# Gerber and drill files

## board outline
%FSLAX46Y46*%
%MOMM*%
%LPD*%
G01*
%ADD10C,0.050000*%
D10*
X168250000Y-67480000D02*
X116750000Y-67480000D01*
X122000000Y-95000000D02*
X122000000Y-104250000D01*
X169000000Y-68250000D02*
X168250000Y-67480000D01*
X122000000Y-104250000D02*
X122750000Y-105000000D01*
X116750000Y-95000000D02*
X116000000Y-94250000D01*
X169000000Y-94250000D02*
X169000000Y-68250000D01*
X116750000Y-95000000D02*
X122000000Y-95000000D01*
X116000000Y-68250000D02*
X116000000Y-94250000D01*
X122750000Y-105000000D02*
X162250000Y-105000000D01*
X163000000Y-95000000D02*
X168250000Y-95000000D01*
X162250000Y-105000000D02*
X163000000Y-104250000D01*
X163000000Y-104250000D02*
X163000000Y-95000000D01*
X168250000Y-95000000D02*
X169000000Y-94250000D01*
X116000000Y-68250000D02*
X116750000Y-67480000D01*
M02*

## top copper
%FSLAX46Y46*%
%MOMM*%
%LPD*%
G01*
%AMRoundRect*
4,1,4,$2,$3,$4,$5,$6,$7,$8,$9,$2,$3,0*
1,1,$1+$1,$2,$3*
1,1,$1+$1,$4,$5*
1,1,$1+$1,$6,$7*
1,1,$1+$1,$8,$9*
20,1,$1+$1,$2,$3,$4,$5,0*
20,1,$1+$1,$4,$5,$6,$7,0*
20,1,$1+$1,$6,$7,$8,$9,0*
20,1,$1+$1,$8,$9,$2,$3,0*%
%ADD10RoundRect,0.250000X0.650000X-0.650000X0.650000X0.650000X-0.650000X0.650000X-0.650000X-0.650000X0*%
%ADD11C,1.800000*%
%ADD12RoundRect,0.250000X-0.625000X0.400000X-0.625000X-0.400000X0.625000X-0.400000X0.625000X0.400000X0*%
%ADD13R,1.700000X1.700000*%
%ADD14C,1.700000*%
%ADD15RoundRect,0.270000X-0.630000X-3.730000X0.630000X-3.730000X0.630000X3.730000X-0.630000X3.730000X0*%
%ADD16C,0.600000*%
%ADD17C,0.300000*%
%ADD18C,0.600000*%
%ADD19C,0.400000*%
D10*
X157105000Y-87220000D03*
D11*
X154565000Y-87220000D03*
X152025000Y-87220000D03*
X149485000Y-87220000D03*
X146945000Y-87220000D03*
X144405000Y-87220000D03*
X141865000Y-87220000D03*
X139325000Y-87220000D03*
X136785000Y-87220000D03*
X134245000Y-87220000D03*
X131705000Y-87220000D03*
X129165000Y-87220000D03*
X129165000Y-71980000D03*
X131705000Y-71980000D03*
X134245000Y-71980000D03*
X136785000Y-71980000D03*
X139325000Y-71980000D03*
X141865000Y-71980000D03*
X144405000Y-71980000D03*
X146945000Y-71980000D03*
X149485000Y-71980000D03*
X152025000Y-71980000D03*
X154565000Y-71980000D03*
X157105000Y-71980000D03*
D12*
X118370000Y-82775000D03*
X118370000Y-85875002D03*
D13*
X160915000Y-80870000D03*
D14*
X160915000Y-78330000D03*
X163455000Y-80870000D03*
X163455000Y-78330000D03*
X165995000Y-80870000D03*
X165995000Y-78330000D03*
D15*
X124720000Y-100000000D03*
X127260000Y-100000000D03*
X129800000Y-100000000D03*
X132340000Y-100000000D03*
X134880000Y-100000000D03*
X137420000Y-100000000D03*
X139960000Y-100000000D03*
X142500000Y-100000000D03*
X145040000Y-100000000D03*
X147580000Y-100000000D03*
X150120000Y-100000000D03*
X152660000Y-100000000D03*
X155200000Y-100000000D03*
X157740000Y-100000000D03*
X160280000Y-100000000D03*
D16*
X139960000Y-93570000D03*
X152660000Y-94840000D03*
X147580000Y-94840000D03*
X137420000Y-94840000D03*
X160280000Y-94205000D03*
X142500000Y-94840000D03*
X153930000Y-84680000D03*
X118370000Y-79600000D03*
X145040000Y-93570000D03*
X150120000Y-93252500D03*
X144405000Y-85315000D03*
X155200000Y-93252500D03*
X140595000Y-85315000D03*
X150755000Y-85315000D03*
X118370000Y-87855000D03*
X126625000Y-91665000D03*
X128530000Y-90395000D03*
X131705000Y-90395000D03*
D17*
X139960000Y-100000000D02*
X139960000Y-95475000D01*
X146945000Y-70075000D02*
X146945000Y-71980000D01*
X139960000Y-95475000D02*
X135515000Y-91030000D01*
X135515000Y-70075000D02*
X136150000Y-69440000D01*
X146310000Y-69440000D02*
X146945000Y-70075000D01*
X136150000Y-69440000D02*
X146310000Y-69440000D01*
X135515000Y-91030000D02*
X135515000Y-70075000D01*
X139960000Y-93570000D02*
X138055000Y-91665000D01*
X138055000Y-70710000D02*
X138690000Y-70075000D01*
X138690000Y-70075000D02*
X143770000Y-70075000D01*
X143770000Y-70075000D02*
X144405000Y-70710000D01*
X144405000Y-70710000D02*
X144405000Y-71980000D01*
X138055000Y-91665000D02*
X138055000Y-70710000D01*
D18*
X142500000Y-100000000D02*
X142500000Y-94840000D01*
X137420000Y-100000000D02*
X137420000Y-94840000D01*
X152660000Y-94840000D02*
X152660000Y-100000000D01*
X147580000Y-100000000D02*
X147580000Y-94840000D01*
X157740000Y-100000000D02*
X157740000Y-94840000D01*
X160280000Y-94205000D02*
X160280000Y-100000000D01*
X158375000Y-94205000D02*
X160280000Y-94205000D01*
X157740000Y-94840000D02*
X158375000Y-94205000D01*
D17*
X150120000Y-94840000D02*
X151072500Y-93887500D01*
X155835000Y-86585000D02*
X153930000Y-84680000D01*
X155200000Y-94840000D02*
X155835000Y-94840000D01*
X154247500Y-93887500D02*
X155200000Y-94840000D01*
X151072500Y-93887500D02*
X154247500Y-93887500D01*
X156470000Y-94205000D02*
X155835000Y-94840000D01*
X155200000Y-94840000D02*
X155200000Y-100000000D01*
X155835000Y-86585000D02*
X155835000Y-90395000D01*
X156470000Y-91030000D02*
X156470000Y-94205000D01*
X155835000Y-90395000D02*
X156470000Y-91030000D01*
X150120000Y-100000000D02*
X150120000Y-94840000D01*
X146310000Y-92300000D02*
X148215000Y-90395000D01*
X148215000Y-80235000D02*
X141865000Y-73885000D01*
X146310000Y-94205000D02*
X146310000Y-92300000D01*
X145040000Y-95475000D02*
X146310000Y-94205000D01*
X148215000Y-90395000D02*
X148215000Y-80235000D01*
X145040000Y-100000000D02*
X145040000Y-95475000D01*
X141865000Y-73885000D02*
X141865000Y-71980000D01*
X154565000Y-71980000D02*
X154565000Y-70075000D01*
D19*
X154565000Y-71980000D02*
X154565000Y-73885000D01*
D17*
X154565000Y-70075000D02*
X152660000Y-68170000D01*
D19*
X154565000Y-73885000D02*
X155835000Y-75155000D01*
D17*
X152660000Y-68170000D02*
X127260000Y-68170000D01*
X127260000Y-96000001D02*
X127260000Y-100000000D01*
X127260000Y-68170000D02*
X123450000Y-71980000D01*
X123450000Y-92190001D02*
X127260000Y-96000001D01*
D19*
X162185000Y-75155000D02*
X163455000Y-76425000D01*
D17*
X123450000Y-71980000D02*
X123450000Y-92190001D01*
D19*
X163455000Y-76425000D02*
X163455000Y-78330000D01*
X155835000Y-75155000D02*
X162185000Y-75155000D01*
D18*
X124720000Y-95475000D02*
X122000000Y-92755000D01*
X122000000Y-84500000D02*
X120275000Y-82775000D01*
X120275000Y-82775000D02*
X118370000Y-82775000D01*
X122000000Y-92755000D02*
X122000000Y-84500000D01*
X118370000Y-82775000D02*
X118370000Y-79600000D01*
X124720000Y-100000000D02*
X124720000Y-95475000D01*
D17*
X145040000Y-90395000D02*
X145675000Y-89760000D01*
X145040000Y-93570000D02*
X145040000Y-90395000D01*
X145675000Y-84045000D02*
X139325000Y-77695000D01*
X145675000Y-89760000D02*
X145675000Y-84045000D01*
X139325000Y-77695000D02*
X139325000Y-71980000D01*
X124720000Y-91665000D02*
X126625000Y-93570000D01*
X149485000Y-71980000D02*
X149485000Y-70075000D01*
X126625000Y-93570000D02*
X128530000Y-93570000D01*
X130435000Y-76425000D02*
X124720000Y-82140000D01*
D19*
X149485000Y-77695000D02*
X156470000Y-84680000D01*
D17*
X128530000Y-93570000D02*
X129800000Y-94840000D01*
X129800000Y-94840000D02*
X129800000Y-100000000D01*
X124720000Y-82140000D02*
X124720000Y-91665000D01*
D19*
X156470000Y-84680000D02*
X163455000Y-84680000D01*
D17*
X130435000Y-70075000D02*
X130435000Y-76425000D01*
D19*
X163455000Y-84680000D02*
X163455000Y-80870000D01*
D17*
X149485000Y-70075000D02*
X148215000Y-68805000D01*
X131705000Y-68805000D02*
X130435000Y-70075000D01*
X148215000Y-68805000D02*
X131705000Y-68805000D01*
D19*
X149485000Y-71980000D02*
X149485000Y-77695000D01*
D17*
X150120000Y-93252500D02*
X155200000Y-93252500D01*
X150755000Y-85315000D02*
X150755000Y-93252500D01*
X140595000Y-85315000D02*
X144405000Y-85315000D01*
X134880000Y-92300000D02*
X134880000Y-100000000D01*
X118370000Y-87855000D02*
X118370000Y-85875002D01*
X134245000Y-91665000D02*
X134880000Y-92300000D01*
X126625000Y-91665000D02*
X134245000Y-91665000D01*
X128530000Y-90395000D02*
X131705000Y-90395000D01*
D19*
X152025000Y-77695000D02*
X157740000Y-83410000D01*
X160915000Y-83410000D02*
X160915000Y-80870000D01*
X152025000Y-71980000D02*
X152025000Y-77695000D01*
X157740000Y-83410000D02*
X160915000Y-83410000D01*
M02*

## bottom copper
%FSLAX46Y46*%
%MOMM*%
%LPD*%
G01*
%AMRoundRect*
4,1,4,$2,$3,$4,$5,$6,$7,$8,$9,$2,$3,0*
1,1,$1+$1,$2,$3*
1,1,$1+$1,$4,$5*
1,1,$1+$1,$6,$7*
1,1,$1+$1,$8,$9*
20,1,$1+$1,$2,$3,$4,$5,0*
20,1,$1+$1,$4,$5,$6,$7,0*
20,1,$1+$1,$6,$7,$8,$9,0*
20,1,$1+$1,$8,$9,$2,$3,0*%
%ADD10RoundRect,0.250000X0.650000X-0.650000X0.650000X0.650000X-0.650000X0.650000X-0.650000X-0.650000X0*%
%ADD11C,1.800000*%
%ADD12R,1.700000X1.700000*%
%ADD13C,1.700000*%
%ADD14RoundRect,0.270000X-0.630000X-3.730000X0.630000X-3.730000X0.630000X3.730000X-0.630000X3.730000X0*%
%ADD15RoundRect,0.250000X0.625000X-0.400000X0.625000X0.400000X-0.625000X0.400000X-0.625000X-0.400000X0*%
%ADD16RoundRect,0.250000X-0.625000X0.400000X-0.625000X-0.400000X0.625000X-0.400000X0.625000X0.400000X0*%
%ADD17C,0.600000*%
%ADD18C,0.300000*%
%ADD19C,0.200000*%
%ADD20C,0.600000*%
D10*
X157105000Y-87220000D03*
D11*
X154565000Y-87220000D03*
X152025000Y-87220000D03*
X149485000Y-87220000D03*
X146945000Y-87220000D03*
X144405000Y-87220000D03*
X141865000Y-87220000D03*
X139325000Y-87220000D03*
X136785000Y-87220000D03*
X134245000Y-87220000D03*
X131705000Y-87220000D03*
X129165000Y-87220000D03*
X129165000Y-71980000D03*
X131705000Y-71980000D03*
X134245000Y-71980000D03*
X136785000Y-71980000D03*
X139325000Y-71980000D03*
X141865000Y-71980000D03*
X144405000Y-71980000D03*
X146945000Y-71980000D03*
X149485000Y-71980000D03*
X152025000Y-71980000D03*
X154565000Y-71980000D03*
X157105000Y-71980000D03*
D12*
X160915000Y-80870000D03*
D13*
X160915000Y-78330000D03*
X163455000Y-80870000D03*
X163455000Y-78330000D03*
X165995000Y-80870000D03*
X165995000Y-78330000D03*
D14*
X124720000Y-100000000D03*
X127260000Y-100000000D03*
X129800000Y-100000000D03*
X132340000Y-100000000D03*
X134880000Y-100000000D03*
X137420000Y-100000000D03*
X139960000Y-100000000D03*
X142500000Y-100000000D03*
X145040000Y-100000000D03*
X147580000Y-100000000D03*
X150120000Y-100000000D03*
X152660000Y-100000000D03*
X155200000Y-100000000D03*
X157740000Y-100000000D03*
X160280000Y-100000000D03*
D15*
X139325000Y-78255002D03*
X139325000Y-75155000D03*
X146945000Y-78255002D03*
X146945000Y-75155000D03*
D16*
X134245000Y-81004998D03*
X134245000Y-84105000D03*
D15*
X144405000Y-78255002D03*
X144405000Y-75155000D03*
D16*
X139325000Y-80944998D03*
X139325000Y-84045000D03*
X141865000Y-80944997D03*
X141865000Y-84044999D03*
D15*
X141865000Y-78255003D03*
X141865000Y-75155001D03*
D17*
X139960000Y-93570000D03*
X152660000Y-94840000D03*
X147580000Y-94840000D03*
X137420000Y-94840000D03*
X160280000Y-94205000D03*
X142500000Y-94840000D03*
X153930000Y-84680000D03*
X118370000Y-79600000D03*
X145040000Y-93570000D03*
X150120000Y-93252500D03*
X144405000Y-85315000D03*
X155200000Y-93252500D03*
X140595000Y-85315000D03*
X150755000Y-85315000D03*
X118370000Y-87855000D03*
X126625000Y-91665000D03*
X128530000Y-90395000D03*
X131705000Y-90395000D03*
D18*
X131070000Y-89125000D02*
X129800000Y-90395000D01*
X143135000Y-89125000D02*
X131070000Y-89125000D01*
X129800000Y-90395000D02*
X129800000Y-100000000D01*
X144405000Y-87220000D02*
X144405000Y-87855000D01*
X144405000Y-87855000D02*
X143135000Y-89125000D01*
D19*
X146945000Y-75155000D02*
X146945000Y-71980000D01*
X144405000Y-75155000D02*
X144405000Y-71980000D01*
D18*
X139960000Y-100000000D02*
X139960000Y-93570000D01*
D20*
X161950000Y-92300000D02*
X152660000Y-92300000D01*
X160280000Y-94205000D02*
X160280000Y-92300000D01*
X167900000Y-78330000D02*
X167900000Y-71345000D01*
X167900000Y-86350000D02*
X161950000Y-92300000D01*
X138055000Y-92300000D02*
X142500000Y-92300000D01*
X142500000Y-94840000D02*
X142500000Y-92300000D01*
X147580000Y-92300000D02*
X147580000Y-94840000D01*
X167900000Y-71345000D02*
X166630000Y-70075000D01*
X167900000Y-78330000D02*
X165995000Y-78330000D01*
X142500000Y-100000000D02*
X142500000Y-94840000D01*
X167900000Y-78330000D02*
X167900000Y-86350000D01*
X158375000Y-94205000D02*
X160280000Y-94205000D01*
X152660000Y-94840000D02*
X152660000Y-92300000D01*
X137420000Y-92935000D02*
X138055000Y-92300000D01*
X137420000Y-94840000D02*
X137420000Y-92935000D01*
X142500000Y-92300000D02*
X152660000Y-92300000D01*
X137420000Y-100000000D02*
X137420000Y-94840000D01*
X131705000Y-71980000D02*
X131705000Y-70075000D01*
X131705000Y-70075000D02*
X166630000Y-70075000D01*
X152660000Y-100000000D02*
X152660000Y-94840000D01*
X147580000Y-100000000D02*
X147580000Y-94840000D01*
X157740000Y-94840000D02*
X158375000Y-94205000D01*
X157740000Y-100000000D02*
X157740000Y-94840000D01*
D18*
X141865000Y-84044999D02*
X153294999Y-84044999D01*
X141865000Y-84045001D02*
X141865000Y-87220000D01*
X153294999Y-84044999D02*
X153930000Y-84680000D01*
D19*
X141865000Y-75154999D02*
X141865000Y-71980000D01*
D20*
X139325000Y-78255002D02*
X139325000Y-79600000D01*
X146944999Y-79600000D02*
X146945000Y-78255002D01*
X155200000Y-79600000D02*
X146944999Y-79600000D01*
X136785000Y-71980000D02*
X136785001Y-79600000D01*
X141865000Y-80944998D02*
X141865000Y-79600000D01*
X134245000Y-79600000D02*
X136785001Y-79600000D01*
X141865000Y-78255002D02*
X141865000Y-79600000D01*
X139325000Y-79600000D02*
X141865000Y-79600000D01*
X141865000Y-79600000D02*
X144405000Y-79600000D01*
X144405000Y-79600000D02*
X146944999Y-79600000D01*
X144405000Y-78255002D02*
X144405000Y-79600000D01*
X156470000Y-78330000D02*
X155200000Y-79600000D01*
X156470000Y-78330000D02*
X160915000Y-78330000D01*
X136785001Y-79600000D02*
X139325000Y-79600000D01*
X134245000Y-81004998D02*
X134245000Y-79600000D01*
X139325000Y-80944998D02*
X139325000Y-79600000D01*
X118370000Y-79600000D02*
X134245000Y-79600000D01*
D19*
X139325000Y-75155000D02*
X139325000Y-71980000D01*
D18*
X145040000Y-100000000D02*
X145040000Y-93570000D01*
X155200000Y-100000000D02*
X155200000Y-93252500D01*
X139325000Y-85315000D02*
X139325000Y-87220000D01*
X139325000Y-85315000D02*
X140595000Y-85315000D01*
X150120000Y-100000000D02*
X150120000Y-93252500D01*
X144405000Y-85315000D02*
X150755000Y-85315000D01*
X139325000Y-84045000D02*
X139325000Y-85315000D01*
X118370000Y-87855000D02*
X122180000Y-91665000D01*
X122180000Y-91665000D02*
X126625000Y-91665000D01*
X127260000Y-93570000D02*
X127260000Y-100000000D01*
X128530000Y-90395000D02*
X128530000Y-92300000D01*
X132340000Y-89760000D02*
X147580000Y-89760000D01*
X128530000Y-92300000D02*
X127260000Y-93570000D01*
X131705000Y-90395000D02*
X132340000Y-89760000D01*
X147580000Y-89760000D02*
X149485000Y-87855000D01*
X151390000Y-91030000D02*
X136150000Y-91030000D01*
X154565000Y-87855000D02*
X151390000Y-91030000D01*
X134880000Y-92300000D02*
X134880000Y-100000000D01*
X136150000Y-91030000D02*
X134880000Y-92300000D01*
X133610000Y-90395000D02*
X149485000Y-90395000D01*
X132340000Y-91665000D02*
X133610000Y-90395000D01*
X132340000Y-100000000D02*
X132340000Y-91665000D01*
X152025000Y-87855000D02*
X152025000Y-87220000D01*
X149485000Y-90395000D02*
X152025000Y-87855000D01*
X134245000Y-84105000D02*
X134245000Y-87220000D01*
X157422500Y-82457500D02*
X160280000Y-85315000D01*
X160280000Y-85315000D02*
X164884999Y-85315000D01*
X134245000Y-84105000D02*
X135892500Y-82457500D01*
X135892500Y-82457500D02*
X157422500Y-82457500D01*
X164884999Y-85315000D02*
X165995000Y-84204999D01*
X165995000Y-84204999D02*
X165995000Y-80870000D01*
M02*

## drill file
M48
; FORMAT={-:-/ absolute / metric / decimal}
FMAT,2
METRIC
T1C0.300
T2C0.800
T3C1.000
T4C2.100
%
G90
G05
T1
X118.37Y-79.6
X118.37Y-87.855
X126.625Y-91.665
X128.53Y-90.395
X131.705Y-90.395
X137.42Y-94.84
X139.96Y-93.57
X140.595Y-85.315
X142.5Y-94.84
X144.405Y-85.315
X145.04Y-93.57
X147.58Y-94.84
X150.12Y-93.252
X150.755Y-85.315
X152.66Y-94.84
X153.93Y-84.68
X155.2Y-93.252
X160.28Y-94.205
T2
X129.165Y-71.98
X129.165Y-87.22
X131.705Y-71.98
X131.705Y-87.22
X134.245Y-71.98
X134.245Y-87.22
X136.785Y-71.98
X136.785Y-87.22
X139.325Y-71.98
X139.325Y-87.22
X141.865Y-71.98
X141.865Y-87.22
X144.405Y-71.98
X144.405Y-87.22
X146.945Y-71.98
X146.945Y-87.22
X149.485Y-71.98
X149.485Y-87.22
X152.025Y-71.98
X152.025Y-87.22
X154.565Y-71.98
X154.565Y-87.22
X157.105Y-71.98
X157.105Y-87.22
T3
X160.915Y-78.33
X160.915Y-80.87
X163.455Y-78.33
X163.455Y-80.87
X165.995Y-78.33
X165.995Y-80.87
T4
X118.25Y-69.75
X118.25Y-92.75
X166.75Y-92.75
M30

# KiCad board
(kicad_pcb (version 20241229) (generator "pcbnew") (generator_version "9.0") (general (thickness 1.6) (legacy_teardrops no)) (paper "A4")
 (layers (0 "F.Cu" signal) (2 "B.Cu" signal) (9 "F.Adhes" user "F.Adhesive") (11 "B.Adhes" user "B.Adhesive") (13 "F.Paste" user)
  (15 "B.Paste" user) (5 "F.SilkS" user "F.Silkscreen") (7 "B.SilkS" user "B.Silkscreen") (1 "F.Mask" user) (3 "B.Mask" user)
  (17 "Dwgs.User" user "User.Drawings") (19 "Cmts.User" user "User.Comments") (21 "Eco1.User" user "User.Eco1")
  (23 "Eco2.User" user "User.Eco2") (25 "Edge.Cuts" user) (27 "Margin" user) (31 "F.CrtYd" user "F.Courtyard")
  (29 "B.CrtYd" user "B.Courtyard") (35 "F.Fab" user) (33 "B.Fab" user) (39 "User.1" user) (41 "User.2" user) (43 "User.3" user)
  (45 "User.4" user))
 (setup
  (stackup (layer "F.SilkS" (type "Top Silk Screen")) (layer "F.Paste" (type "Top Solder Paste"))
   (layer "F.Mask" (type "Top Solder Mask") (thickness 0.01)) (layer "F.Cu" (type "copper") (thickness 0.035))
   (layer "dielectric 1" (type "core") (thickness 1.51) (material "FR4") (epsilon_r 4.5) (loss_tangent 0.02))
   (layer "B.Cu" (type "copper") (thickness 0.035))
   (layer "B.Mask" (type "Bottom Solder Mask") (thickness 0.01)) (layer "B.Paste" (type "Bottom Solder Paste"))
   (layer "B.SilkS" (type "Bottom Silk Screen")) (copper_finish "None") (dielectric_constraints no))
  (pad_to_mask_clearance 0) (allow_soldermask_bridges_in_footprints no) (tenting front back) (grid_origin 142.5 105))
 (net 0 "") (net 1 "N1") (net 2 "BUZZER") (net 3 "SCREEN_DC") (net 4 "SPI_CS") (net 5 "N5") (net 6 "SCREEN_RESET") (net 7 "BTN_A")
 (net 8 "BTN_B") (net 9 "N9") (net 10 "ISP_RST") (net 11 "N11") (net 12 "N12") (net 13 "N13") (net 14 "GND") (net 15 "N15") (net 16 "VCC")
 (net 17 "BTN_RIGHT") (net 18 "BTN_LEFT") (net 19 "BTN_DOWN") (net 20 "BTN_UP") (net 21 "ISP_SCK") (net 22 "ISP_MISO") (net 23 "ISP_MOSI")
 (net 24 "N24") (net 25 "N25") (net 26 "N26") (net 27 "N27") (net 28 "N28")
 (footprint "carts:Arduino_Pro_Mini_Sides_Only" (layer "F.Cu") (at 141.865 79.6 90)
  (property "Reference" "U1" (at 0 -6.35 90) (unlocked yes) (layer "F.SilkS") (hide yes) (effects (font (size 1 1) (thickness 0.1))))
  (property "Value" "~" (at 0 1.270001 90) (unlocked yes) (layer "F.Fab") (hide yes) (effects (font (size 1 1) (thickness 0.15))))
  (pad "1" thru_hole roundrect (at -7.62 15.24 90) (size 1.8 1.8) (drill 0.8) (layers "*.Cu" "*.Mask") (remove_unused_layers no)
   (roundrect_rratio 0.1388888889) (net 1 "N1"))
  (pad "2" thru_hole circle (at -7.62 12.7 90) (size 1.8 1.8) (drill 0.8) (layers "*.Cu" "*.Mask") (remove_unused_layers no)
   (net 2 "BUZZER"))
  (pad "3" thru_hole circle (at -7.62 10.16 90) (size 1.8 1.8) (drill 0.8) (layers "*.Cu" "*.Mask") (remove_unused_layers no)
   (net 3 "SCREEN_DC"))
  (pad "4" thru_hole circle (at -7.62 7.62 90) (size 1.8 1.8) (drill 0.8) (layers "*.Cu" "*.Mask") (remove_unused_layers no)
   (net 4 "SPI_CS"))
  (pad "5" thru_hole circle (at -7.62 5.08 90) (size 1.8 1.8) (drill 0.8) (layers "*.Cu" "*.Mask") (remove_unused_layers no) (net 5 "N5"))
  (pad "6" thru_hole circle (at -7.62 2.54 90) (size 1.8 1.8) (drill 0.8) (layers "*.Cu" "*.Mask") (remove_unused_layers no)
   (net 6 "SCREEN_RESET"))
  (pad "7" thru_hole circle (at -7.62 0 90) (size 1.8 1.8) (drill 0.8) (layers "*.Cu" "*.Mask") (remove_unused_layers no) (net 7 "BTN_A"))
  (pad "8" thru_hole circle (at -7.62 -2.54 90) (size 1.8 1.8) (drill 0.8) (layers "*.Cu" "*.Mask") (remove_unused_layers no)
   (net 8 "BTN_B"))
  (pad "9" thru_hole circle (at -7.62 -5.08 90) (size 1.8 1.8) (drill 0.8) (layers "*.Cu" "*.Mask") (remove_unused_layers no) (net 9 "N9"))
  (pad "10" thru_hole circle (at -7.62 -7.62 90) (size 1.8 1.8) (drill 0.8) (layers "*.Cu" "*.Mask") (remove_unused_layers no)
   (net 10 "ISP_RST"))
  (pad "11" thru_hole circle (at -7.62 -10.16 90) (size 1.8 1.8) (drill 0.8) (layers "*.Cu" "*.Mask") (remove_unused_layers no)
   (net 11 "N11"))
  (pad "12" thru_hole circle (at -7.62 -12.7 90) (size 1.8 1.8) (drill 0.8) (layers "*.Cu" "*.Mask") (remove_unused_layers no)
   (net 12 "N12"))
  (pad "19" thru_hole circle (at 7.62 -12.7 90) (size 1.8 1.8) (drill 0.8) (layers "*.Cu" "*.Mask") (remove_unused_layers no) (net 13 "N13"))
  (pad "20" thru_hole circle (at 7.62 -10.16 90) (size 1.8 1.8) (drill 0.8) (layers "*.Cu" "*.Mask") (remove_unused_layers no)
   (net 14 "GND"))
  (pad "21" thru_hole circle (at 7.62 -7.62 90) (size 1.8 1.8) (drill 0.8) (layers "*.Cu" "*.Mask") (remove_unused_layers no) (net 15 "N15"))
  (pad "22" thru_hole circle (at 7.62 -5.08 90) (size 1.8 1.8) (drill 0.8) (layers "*.Cu" "*.Mask") (remove_unused_layers no) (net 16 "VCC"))
  (pad "23" thru_hole circle (at 7.62 -2.54 90) (size 1.8 1.8) (drill 0.8) (layers "*.Cu" "*.Mask") (remove_unused_layers no)
   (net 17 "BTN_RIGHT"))
  (pad "24" thru_hole circle (at 7.62 0 90) (size 1.8 1.8) (drill 0.8) (layers "*.Cu" "*.Mask") (remove_unused_layers no)
   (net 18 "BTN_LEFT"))
  (pad "25" thru_hole circle (at 7.62 2.54 90) (size 1.8 1.8) (drill 0.8) (layers "*.Cu" "*.Mask") (remove_unused_layers no)
   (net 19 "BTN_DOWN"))
  (pad "26" thru_hole circle (at 7.62 5.08 90) (size 1.8 1.8) (drill 0.8) (layers "*.Cu" "*.Mask") (remove_unused_layers no)
   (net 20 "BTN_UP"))
  (pad "27" thru_hole circle (at 7.62 7.62 90) (size 1.8 1.8) (drill 0.8) (layers "*.Cu" "*.Mask") (remove_unused_layers no)
   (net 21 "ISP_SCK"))
  (pad "28" thru_hole circle (at 7.62 10.16 90) (size 1.8 1.8) (drill 0.8) (layers "*.Cu" "*.Mask") (remove_unused_layers no)
   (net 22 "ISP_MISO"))
  (pad "29" thru_hole circle (at 7.62 12.7 90) (size 1.8 1.8) (drill 0.8) (layers "*.Cu" "*.Mask") (remove_unused_layers no)
   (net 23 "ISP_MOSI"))
  (pad "30" thru_hole circle (at 7.62 15.24 90) (size 1.8 1.8) (drill 0.8) (layers "*.Cu" "*.Mask") (remove_unused_layers no) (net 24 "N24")))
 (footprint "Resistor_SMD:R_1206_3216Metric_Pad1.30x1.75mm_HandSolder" (layer "F.Cu") (at 118.37 84.325001 -90)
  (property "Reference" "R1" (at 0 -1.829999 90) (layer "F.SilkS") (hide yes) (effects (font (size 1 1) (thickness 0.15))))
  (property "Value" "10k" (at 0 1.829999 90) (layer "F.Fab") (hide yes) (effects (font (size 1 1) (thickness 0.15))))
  (pad "1" smd roundrect (at -1.550001 0 270) (size 1.3 1.75) (layers "F.Cu" "F.Mask" "F.Paste") (roundrect_rratio 0.192308) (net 16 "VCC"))
  (pad "2" smd roundrect (at 1.550001 0 270) (size 1.3 1.75) (layers "F.Cu" "F.Mask" "F.Paste") (roundrect_rratio 0.192308) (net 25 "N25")))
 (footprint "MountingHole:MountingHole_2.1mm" (layer "F.Cu") (at 118.25 92.75)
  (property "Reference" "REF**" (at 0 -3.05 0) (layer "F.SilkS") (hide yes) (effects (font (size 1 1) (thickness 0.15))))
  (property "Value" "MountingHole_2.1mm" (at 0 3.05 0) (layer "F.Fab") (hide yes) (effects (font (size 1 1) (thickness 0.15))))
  (pad "" np_thru_hole circle (at 0 0) (size 2.1 2.1) (drill 2.1) (layers "*.Cu" "*.Mask")))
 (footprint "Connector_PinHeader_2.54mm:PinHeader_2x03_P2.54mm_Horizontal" (layer "F.Cu") (at 160.915 80.87 90)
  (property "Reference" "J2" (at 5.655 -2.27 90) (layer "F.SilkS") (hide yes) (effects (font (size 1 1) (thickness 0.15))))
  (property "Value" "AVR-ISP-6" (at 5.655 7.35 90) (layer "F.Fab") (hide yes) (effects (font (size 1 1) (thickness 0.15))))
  (pad "1" thru_hole rect (at 0 0 90) (size 1.7 1.7) (drill 1) (layers "*.Cu" "*.Mask") (remove_unused_layers no) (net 22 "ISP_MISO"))
  (pad "2" thru_hole circle (at 2.54 0 90) (size 1.7 1.7) (drill 1) (layers "*.Cu" "*.Mask") (remove_unused_layers no) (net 16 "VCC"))
  (pad "3" thru_hole circle (at 0 2.54 90) (size 1.7 1.7) (drill 1) (layers "*.Cu" "*.Mask") (remove_unused_layers no) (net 21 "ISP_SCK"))
  (pad "4" thru_hole circle (at 2.54 2.54 90) (size 1.7 1.7) (drill 1) (layers "*.Cu" "*.Mask") (remove_unused_layers no)
   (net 23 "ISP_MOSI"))
  (pad "5" thru_hole circle (at 0 5.08 90) (size 1.7 1.7) (drill 1) (layers "*.Cu" "*.Mask") (remove_unused_layers no) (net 10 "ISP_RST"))
  (pad "6" thru_hole circle (at 2.54 5.08 90) (size 1.7 1.7) (drill 1) (layers "*.Cu" "*.Mask") (remove_unused_layers no) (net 14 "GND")))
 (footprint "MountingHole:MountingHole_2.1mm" (layer "F.Cu") (at 118.25 69.75)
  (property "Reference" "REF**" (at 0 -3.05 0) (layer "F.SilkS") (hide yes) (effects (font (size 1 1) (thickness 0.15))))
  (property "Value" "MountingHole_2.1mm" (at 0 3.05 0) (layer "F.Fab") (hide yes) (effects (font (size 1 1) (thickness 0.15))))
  (pad "" np_thru_hole circle (at 0 0) (size 2.1 2.1) (drill 2.1) (layers "*.Cu" "*.Mask")))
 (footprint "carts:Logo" (layer "F.Cu") (at 122.75 75.75)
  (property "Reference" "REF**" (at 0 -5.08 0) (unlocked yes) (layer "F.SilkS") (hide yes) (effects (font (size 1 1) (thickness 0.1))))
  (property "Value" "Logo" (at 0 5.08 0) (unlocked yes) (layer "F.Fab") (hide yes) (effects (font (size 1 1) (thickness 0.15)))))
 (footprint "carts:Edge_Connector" (layer "F.Cu") (at 142.5 100)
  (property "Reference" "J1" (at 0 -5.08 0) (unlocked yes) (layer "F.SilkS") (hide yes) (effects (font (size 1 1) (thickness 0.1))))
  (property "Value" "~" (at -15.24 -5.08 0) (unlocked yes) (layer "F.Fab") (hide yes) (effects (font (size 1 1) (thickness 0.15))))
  (pad "1" connect roundrect (at -17.78 0) (size 1.8 8) (layers "F.Cu" "F.Mask") (roundrect_rratio 0.15) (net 16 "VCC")
   (thermal_bridge_angle 45))
  (pad "2" connect roundrect (at -17.78 0) (size 1.8 8) (layers "B.Cu" "B.Mask") (roundrect_rratio 0.15) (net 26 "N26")
   (thermal_bridge_angle 45))
  (pad "3" connect roundrect (at -15.24 0) (size 1.8 8) (layers "F.Cu" "F.Mask") (roundrect_rratio 0.15) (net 23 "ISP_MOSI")
   (thermal_bridge_angle 45))
  (pad "4" connect roundrect (at -15.24 0) (size 1.8 8) (layers "B.Cu" "B.Mask") (roundrect_rratio 0.15) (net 4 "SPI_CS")
   (thermal_bridge_angle 45))
  (pad "5" connect roundrect (at -12.7 0) (size 1.8 8) (layers "F.Cu" "F.Mask") (roundrect_rratio 0.15) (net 21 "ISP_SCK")
   (thermal_bridge_angle 45))
  (pad "6" connect roundrect (at -12.7 0) (size 1.8 8) (layers "B.Cu" "B.Mask") (roundrect_rratio 0.15) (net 6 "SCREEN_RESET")
   (thermal_bridge_angle 45))
  (pad "7" connect roundrect (at -10.16 0) (size 1.8 8) (layers "F.Cu" "F.Mask") (roundrect_rratio 0.15) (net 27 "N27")
   (thermal_bridge_angle 45))
  (pad "8" connect roundrect (at -10.16 0) (size 1.8 8) (layers "B.Cu" "B.Mask") (roundrect_rratio 0.15) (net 3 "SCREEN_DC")
   (thermal_bridge_angle 45))
  (pad "9" connect roundrect (at -7.62 0) (size 1.8 8) (layers "F.Cu" "F.Mask") (roundrect_rratio 0.15) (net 25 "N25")
   (thermal_bridge_angle 45))
  (pad "10" connect roundrect (at -7.62 0) (size 1.8 8) (layers "B.Cu" "B.Mask") (roundrect_rratio 0.15) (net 2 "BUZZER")
   (thermal_bridge_angle 45))
  (pad "11" connect roundrect (at -5.08 0) (size 1.8 8) (layers "F.Cu" "F.Mask") (roundrect_rratio 0.15) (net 14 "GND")
   (thermal_bridge_angle 45))
  (pad "12" connect roundrect (at -5.08 0) (size 1.8 8) (layers "B.Cu" "B.Mask") (roundrect_rratio 0.15) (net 14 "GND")
   (thermal_bridge_angle 45))
  (pad "13" connect roundrect (at -2.54 0) (size 1.8 8) (layers "F.Cu" "F.Mask") (roundrect_rratio 0.15) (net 20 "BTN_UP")
   (thermal_bridge_angle 45))
  (pad "14" connect roundrect (at -2.54 0) (size 1.8 8) (layers "B.Cu" "B.Mask") (roundrect_rratio 0.15) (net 19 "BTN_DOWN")
   (thermal_bridge_angle 45))
  (pad "15" connect roundrect (at 0 0) (size 1.8 8) (layers "F.Cu" "F.Mask") (roundrect_rratio 0.15) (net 14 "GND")
   (thermal_bridge_angle 45))
  (pad "16" connect roundrect (at 0 0) (size 1.8 8) (layers "B.Cu" "B.Mask") (roundrect_rratio 0.15) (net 14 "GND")
   (thermal_bridge_angle 45))
  (pad "17" connect roundrect (at 2.54 0) (size 1.8 8) (layers "F.Cu" "F.Mask") (roundrect_rratio 0.15) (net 18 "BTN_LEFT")
   (thermal_bridge_angle 45))
  (pad "18" connect roundrect (at 2.54 0) (size 1.8 8) (layers "B.Cu" "B.Mask") (roundrect_rratio 0.15) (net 17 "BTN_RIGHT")
   (thermal_bridge_angle 45))
  (pad "19" connect roundrect (at 5.08 0) (size 1.8 8) (layers "F.Cu" "F.Mask") (roundrect_rratio 0.15) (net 14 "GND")
   (thermal_bridge_angle 45))
  (pad "20" connect roundrect (at 5.08 0) (size 1.8 8) (layers "B.Cu" "B.Mask") (roundrect_rratio 0.15) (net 14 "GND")
   (thermal_bridge_angle 45))
  (pad "21" connect roundrect (at 7.62 0) (size 1.8 8) (layers "F.Cu" "F.Mask") (roundrect_rratio 0.15) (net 7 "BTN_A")
   (thermal_bridge_angle 45))
  (pad "22" connect roundrect (at 7.62 0) (size 1.8 8) (layers "B.Cu" "B.Mask") (roundrect_rratio 0.15) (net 8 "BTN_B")
   (thermal_bridge_angle 45))
  (pad "23" connect roundrect (at 10.16 0) (size 1.8 8) (layers "F.Cu" "F.Mask") (roundrect_rratio 0.15) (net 14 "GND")
   (thermal_bridge_angle 45))
  (pad "24" connect roundrect (at 10.16 0) (size 1.8 8) (layers "B.Cu" "B.Mask") (roundrect_rratio 0.15) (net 14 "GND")
   (thermal_bridge_angle 45))
  (pad "25" connect roundrect (at 12.7 0) (size 1.8 8) (layers "F.Cu" "F.Mask") (roundrect_rratio 0.15) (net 7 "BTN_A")
   (thermal_bridge_angle 45))
  (pad "26" connect roundrect (at 12.7 0) (size 1.8 8) (layers "B.Cu" "B.Mask") (roundrect_rratio 0.15) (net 8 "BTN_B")
   (thermal_bridge_angle 45))
  (pad "27" connect roundrect (at 15.24 0) (size 1.8 8) (layers "F.Cu" "F.Mask") (roundrect_rratio 0.15) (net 14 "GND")
   (thermal_bridge_angle 45))
  (pad "28" connect roundrect (at 15.24 0) (size 1.8 8) (layers "B.Cu" "B.Mask") (roundrect_rratio 0.15) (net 14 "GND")
   (thermal_bridge_angle 45))
  (pad "29" connect roundrect (at 17.78 0) (size 1.8 8) (layers "F.Cu" "F.Mask") (roundrect_rratio 0.15) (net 14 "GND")
   (thermal_bridge_angle 45))
  (pad "30" connect roundrect (at 17.78 0) (size 1.8 8) (layers "B.Cu" "B.Mask") (roundrect_rratio 0.15) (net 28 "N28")
   (thermal_bridge_angle 45)))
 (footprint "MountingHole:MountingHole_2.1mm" (layer "F.Cu") (at 166.75 92.75)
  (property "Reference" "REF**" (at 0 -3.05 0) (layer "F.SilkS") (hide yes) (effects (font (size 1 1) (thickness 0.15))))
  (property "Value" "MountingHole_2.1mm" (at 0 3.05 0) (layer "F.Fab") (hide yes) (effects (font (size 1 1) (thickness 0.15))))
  (pad "" np_thru_hole circle (at 0 0) (size 2.1 2.1) (drill 2.1) (layers "*.Cu" "*.Mask")))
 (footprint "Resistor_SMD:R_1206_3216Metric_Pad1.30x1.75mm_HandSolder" (layer "B.Cu") (at 139.325 76.705001 90)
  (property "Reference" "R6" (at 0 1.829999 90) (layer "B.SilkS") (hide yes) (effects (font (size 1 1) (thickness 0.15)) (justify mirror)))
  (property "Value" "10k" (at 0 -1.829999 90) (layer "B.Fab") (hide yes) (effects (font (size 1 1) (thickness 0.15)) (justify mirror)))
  (pad "1" smd roundrect (at -1.550001 0 90) (size 1.3 1.75) (layers "B.Cu" "B.Mask" "B.Paste") (roundrect_rratio 0.192308) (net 16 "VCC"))
  (pad "2" smd roundrect (at 1.550001 0 90) (size 1.3 1.75) (layers "B.Cu" "B.Mask" "B.Paste") (roundrect_rratio 0.192308)
   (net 17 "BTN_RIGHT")))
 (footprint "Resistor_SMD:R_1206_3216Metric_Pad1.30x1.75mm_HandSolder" (layer "B.Cu") (at 146.945 76.705001 90)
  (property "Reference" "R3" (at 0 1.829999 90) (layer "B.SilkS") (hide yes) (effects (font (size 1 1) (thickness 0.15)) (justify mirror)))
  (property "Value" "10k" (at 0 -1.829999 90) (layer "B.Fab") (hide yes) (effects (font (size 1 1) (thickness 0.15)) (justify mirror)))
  (pad "1" smd roundrect (at -1.550001 0 90) (size 1.3 1.75) (layers "B.Cu" "B.Mask" "B.Paste") (roundrect_rratio 0.192308) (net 16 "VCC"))
  (pad "2" smd roundrect (at 1.550001 0 90) (size 1.3 1.75) (layers "B.Cu" "B.Mask" "B.Paste") (roundrect_rratio 0.192308) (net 20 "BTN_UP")))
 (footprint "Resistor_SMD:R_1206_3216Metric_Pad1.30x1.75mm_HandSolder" (layer "B.Cu") (at 134.245 82.554999 -90)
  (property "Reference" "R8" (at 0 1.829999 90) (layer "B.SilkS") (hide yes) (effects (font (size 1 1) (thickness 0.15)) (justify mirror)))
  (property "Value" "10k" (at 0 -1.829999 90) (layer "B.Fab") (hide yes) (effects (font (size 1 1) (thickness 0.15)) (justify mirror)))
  (pad "1" smd roundrect (at -1.550001 0 270) (size 1.3 1.75) (layers "B.Cu" "B.Mask" "B.Paste") (roundrect_rratio 0.192308) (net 16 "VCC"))
  (pad "2" smd roundrect (at 1.550001 0 270) (size 1.3 1.75) (layers "B.Cu" "B.Mask" "B.Paste") (roundrect_rratio 0.192308)
   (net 10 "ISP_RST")))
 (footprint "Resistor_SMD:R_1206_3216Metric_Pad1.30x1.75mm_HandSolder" (layer "B.Cu") (at 144.405 76.705001 90)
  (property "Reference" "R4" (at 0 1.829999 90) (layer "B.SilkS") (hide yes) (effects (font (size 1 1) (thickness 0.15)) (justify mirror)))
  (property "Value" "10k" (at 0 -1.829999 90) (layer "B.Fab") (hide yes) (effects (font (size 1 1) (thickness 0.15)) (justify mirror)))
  (pad "1" smd roundrect (at -1.550001 0 90) (size 1.3 1.75) (layers "B.Cu" "B.Mask" "B.Paste") (roundrect_rratio 0.192308) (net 16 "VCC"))
  (pad "2" smd roundrect (at 1.550001 0 90) (size 1.3 1.75) (layers "B.Cu" "B.Mask" "B.Paste") (roundrect_rratio 0.192308)
   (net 19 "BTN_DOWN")))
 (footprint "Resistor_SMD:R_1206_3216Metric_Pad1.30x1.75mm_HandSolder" (layer "B.Cu") (at 139.325 82.494999 -90)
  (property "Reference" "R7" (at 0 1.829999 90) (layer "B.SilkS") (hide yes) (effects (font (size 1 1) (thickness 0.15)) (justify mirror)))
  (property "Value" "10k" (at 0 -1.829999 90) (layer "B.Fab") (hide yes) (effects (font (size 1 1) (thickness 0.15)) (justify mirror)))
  (pad "1" smd roundrect (at -1.550001 0 270) (size 1.3 1.75) (layers "B.Cu" "B.Mask" "B.Paste") (roundrect_rratio 0.192308) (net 16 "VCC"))
  (pad "2" smd roundrect (at 1.550001 0 270) (size 1.3 1.75) (layers "B.Cu" "B.Mask" "B.Paste") (roundrect_rratio 0.192308) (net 8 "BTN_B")))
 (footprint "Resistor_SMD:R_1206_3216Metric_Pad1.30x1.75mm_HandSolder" (layer "B.Cu") (at 141.865 82.494998 -90)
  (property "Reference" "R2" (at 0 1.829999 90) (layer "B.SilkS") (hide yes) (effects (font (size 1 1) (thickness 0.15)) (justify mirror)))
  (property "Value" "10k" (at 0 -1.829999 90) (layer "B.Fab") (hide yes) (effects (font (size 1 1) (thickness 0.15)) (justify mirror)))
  (pad "1" smd roundrect (at -1.550001 0 270) (size 1.3 1.75) (layers "B.Cu" "B.Mask" "B.Paste") (roundrect_rratio 0.192308) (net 16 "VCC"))
  (pad "2" smd roundrect (at 1.550001 0 270) (size 1.3 1.75) (layers "B.Cu" "B.Mask" "B.Paste") (roundrect_rratio 0.192308) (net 7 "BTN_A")))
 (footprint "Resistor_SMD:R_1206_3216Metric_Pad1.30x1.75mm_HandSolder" (layer "B.Cu") (at 141.865 76.705002 90)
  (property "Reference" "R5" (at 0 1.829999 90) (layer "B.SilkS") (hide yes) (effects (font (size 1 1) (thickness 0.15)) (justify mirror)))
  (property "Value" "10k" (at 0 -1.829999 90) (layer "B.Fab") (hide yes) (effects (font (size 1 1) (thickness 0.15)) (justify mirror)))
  (pad "1" smd roundrect (at -1.550001 0 90) (size 1.3 1.75) (layers "B.Cu" "B.Mask" "B.Paste") (roundrect_rratio 0.192308) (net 16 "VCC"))
  (pad "2" smd roundrect (at 1.550001 0 90) (size 1.3 1.75) (layers "B.Cu" "B.Mask" "B.Paste") (roundrect_rratio 0.192308)
   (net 18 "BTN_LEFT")))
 (gr_line (start 168.25 67.48) (end 116.75 67.48) (stroke (width 0.05) (type default)) (layer "Edge.Cuts"))
 (gr_line (start 122 95) (end 122 104.25) (stroke (width 0.05) (type default)) (layer "Edge.Cuts"))
 (gr_line (start 169 68.25) (end 168.25 67.48) (stroke (width 0.05) (type default)) (layer "Edge.Cuts"))
 (gr_line (start 122 104.25) (end 122.75 105) (stroke (width 0.05) (type default)) (layer "Edge.Cuts"))
 (gr_line (start 116.75 95) (end 116 94.25) (stroke (width 0.05) (type default)) (layer "Edge.Cuts"))
 (gr_line (start 169 94.25) (end 169 68.25) (stroke (width 0.05) (type solid)) (layer "Edge.Cuts"))
 (gr_line (start 116.75 95) (end 122 95) (stroke (width 0.05) (type solid)) (layer "Edge.Cuts"))
 (gr_line (start 116 68.25) (end 116 94.25) (stroke (width 0.05) (type solid)) (layer "Edge.Cuts"))
 (gr_line (start 122.75 105) (end 162.25 105) (stroke (width 0.05) (type default)) (layer "Edge.Cuts"))
 (gr_line (start 163 95) (end 168.25 95) (stroke (width 0.05) (type solid)) (layer "Edge.Cuts"))
 (gr_line (start 162.25 105) (end 163 104.25) (stroke (width 0.05) (type default)) (layer "Edge.Cuts"))
 (gr_line (start 163 104.25) (end 163 95) (stroke (width 0.05) (type default)) (layer "Edge.Cuts"))
 (gr_line (start 168.25 95) (end 169 94.25) (stroke (width 0.05) (type default)) (layer "Edge.Cuts"))
 (gr_line (start 116 68.25) (end 116.75 67.48) (stroke (width 0.05) (type default)) (layer "Edge.Cuts"))
 (segment (start 131.07 89.125) (end 129.8 90.395) (width 0.3) (layer "B.Cu") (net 6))
 (segment (start 143.135 89.125) (end 131.07 89.125) (width 0.3) (layer "B.Cu") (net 6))
 (segment (start 129.8 90.395) (end 129.8 100) (width 0.3) (layer "B.Cu") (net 6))
 (segment (start 144.405 87.22) (end 144.405 87.855) (width 0.3) (layer "B.Cu") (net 6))
 (segment (start 144.405 87.855) (end 143.135 89.125) (width 0.3) (layer "B.Cu") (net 6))
 (segment (start 139.96 100) (end 139.96 95.475) (width 0.3) (layer "F.Cu") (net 20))
 (segment (start 146.945 70.075) (end 146.945 71.98) (width 0.3) (layer "F.Cu") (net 20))
 (segment (start 139.96 95.475) (end 135.515 91.03) (width 0.3) (layer "F.Cu") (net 20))
 (segment (start 135.515 70.075) (end 136.15 69.44) (width 0.3) (layer "F.Cu") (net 20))
 (segment (start 146.31 69.44) (end 146.945 70.075) (width 0.3) (layer "F.Cu") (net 20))
 (segment (start 136.15 69.44) (end 146.31 69.44) (width 0.3) (layer "F.Cu") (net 20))
 (segment (start 135.515 91.03) (end 135.515 70.075) (width 0.3) (layer "F.Cu") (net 20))
 (segment (start 146.945 75.155) (end 146.945 71.98) (width 0.2) (layer "B.Cu") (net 20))
 (segment (start 139.96 93.57) (end 138.055 91.665) (width 0.3) (layer "F.Cu") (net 19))
 (segment (start 138.055 70.71) (end 138.69 70.075) (width 0.3) (layer "F.Cu") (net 19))
 (segment (start 138.69 70.075) (end 143.77 70.075) (width 0.3) (layer "F.Cu") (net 19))
 (segment (start 143.77 70.075) (end 144.405 70.71) (width 0.3) (layer "F.Cu") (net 19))
 (segment (start 144.405 70.71) (end 144.405 71.98) (width 0.3) (layer "F.Cu") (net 19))
 (segment (start 138.055 91.665) (end 138.055 70.71) (width 0.3) (layer "F.Cu") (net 19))
 (via (at 139.96 93.57) (size 0.6) (drill 0.3) (layers "F.Cu" "B.Cu") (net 19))
 (segment (start 144.405 75.155) (end 144.405 71.98) (width 0.2) (layer "B.Cu") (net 19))
 (segment (start 139.96 100) (end 139.96 93.57) (width 0.3) (layer "B.Cu") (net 19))
 (segment (start 142.5 100) (end 142.5 94.84) (width 0.6) (layer "F.Cu") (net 14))
 (segment (start 137.42 100) (end 137.42 94.84) (width 0.6) (layer "F.Cu") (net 14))
 (segment (start 152.66 94.84) (end 152.66 100) (width 0.6) (layer "F.Cu") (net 14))
 (segment (start 147.58 100) (end 147.58 94.84) (width 0.6) (layer "F.Cu") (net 14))
 (segment (start 157.74 100) (end 157.74 94.84) (width 0.6) (layer "F.Cu") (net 14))
 (segment (start 160.28 94.205) (end 160.28 100) (width 0.6) (layer "F.Cu") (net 14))
 (segment (start 158.375 94.205) (end 160.28 94.205) (width 0.6) (layer "F.Cu") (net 14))
 (segment (start 157.74 94.84) (end 158.375 94.205) (width 0.6) (layer "F.Cu") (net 14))
 (via (at 152.66 94.84) (size 0.6) (drill 0.3) (layers "F.Cu" "B.Cu") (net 14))
 (via (at 147.58 94.84) (size 0.6) (drill 0.3) (layers "F.Cu" "B.Cu") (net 14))
 (via (at 137.42 94.84) (size 0.6) (drill 0.3) (layers "F.Cu" "B.Cu") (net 14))
 (via (at 160.28 94.205) (size 0.6) (drill 0.3) (layers "F.Cu" "B.Cu") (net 14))
 (via (at 142.5 94.84) (size 0.6) (drill 0.3) (layers "F.Cu" "B.Cu") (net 14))
 (segment (start 161.95 92.3) (end 152.66 92.3) (width 0.6) (layer "B.Cu") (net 14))
 (segment (start 160.28 94.205) (end 160.28 92.3) (width 0.6) (layer "B.Cu") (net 14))
 (segment (start 167.9 78.33) (end 167.9 71.345) (width 0.6) (layer "B.Cu") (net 14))
 (segment (start 167.9 86.35) (end 161.95 92.3) (width 0.6) (layer "B.Cu") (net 14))
 (segment (start 138.055 92.3) (end 142.5 92.3) (width 0.6) (layer "B.Cu") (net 14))
 (segment (start 142.5 94.84) (end 142.5 92.3) (width 0.6) (layer "B.Cu") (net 14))
 (segment (start 147.58 92.3) (end 147.58 94.84) (width 0.6) (layer "B.Cu") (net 14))
 (segment (start 167.9 71.345) (end 166.63 70.075) (width 0.6) (layer "B.Cu") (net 14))
 (segment (start 167.9 78.33) (end 165.995 78.33) (width 0.6) (layer "B.Cu") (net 14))
 (segment (start 142.5 100) (end 142.5 94.84) (width 0.6) (layer "B.Cu") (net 14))
 (segment (start 167.9 78.33) (end 167.9 86.35) (width 0.6) (layer "B.Cu") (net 14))
 (segment (start 158.375 94.205) (end 160.28 94.205) (width 0.6) (layer "B.Cu") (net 14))
 (segment (start 152.66 94.84) (end 152.66 92.3) (width 0.6) (layer "B.Cu") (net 14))
 (segment (start 137.42 92.935) (end 138.055 92.3) (width 0.6) (layer "B.Cu") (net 14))
 (segment (start 137.42 94.84) (end 137.42 92.935) (width 0.6) (layer "B.Cu") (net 14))
 (segment (start 142.5 92.3) (end 152.66 92.3) (width 0.6) (layer "B.Cu") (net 14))
 (segment (start 137.42 100) (end 137.42 94.84) (width 0.6) (layer "B.Cu") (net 14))
 (segment (start 131.705 71.98) (end 131.705 70.075) (width 0.6) (layer "B.Cu") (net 14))
 (segment (start 131.705 70.075) (end 166.63 70.075) (width 0.6) (layer "B.Cu") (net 14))
 (segment (start 152.66 100) (end 152.66 94.84) (width 0.6) (layer "B.Cu") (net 14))
 (segment (start 147.58 100) (end 147.58 94.84) (width 0.6) (layer "B.Cu") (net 14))
 (segment (start 157.74 94.84) (end 158.375 94.205) (width 0.6) (layer "B.Cu") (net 14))
 (segment (start 157.74 100) (end 157.74 94.84) (width 0.6) (layer "B.Cu") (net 14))
 (segment (start 150.12 94.84) (end 151.0725 93.8875) (width 0.3) (layer "F.Cu") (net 7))
 (segment (start 155.835 86.585) (end 153.93 84.68) (width 0.3) (layer "F.Cu") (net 7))
 (segment (start 155.2 94.84) (end 155.835 94.84) (width 0.3) (layer "F.Cu") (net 7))
 (segment (start 154.2475 93.8875) (end 155.2 94.84) (width 0.3) (layer "F.Cu") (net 7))
 (segment (start 151.0725 93.8875) (end 154.2475 93.8875) (width 0.3) (layer "F.Cu") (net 7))
 (segment (start 156.47 94.205) (end 155.835 94.84) (width 0.3) (layer "F.Cu") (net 7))
 (segment (start 155.2 94.84) (end 155.2 100) (width 0.3) (layer "F.Cu") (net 7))
 (segment (start 155.835 86.585) (end 155.835 90.395) (width 0.3) (layer "F.Cu") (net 7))
 (segment (start 156.47 91.03) (end 156.47 94.205) (width 0.3) (layer "F.Cu") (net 7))
 (segment (start 155.835 90.395) (end 156.47 91.03) (width 0.3) (layer "F.Cu") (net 7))
 (segment (start 150.12 100) (end 150.12 94.84) (width 0.3) (layer "F.Cu") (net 7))
 (via (at 153.93 84.68) (size 0.6) (drill 0.3) (layers "F.Cu" "B.Cu") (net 7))
 (segment (start 141.865 84.044999) (end 153.294999 84.044999) (width 0.3) (layer "B.Cu") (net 7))
 (segment (start 141.865 84.045001) (end 141.865 87.22) (width 0.3) (layer "B.Cu") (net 7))
 (segment (start 153.294999 84.044999) (end 153.93 84.68) (width 0.3) (layer "B.Cu") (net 7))
 (segment (start 146.31 92.3) (end 148.215 90.395) (width 0.3) (layer "F.Cu") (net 18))
 (segment (start 148.215 80.235) (end 141.865 73.885) (width 0.3) (layer "F.Cu") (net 18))
 (segment (start 146.31 94.205) (end 146.31 92.3) (width 0.3) (layer "F.Cu") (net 18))
 (segment (start 145.04 95.475) (end 146.31 94.205) (width 0.3) (layer "F.Cu") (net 18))
 (segment (start 148.215 90.395) (end 148.215 80.235) (width 0.3) (layer "F.Cu") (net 18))
 (segment (start 145.04 100) (end 145.04 95.475) (width 0.3) (layer "F.Cu") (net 18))
 (segment (start 141.865 73.885) (end 141.865 71.98) (width 0.3) (layer "F.Cu") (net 18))
 (segment (start 141.865 75.154999) (end 141.865 71.98) (width 0.2) (layer "B.Cu") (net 18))
 (segment (start 154.565 71.98) (end 154.565 70.075) (width 0.3) (layer "F.Cu") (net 23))
 (segment (start 154.565 71.98) (end 154.565 73.885) (width 0.4) (layer "F.Cu") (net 23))
 (segment (start 154.565 70.075) (end 152.66 68.17) (width 0.3) (layer "F.Cu") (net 23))
 (segment (start 154.565 73.885) (end 155.835 75.155) (width 0.4) (layer "F.Cu") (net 23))
 (segment (start 152.66 68.17) (end 127.26 68.17) (width 0.3) (layer "F.Cu") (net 23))
 (segment (start 127.26 96.000001) (end 127.26 100) (width 0.3) (layer "F.Cu") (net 23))
 (segment (start 127.26 68.17) (end 123.45 71.98) (width 0.3) (layer "F.Cu") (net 23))
 (segment (start 123.45 92.190001) (end 127.26 96.000001) (width 0.3) (layer "F.Cu") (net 23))
 (segment (start 162.185 75.155) (end 163.455 76.425) (width 0.4) (layer "F.Cu") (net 23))
 (segment (start 123.45 71.98) (end 123.45 92.190001) (width 0.3) (layer "F.Cu") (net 23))
 (segment (start 163.455 76.425) (end 163.455 78.33) (width 0.4) (layer "F.Cu") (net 23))
 (segment (start 155.835 75.155) (end 162.185 75.155) (width 0.4) (layer "F.Cu") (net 23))
 (segment (start 124.72 95.475) (end 122 92.755) (width 0.6) (layer "F.Cu") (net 16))
 (segment (start 122 84.5) (end 120.275 82.775) (width 0.6) (layer "F.Cu") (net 16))
 (segment (start 120.275 82.775) (end 118.37 82.775) (width 0.6) (layer "F.Cu") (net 16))
 (segment (start 122 92.755) (end 122 84.5) (width 0.6) (layer "F.Cu") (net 16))
 (segment (start 118.37 82.775) (end 118.37 79.6) (width 0.6) (layer "F.Cu") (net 16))
 (segment (start 124.72 100) (end 124.72 95.475) (width 0.6) (layer "F.Cu") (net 16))
 (via (at 118.37 79.6) (size 0.6) (drill 0.3) (layers "F.Cu" "B.Cu") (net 16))
 (segment (start 139.325 78.255002) (end 139.325 79.6) (width 0.6) (layer "B.Cu") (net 16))
 (segment (start 146.944999 79.6) (end 146.945 78.255002) (width 0.6) (layer "B.Cu") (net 16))
 (segment (start 155.2 79.6) (end 146.944999 79.6) (width 0.6) (layer "B.Cu") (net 16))
 (segment (start 136.785 71.98) (end 136.785001 79.6) (width 0.6) (layer "B.Cu") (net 16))
 (segment (start 141.865 80.944998) (end 141.865 79.6) (width 0.6) (layer "B.Cu") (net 16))
 (segment (start 134.245 79.6) (end 136.785001 79.6) (width 0.6) (layer "B.Cu") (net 16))
 (segment (start 141.865 78.255002) (end 141.865 79.6) (width 0.6) (layer "B.Cu") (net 16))
 (segment (start 139.325 79.6) (end 141.865 79.6) (width 0.6) (layer "B.Cu") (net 16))
 (segment (start 141.865 79.6) (end 144.405 79.6) (width 0.6) (layer "B.Cu") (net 16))
 (segment (start 144.405 79.6) (end 146.944999 79.6) (width 0.6) (layer "B.Cu") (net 16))
 (segment (start 144.405 78.255002) (end 144.405 79.6) (width 0.6) (layer "B.Cu") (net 16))
 (segment (start 156.47 78.33) (end 155.2 79.6) (width 0.6) (layer "B.Cu") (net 16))
 (segment (start 156.47 78.33) (end 160.915 78.33) (width 0.6) (layer "B.Cu") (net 16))
 (segment (start 136.785001 79.6) (end 139.325 79.6) (width 0.6) (layer "B.Cu") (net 16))
 (segment (start 134.245 81.004998) (end 134.245 79.6) (width 0.6) (layer "B.Cu") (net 16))
 (segment (start 139.325 80.944998) (end 139.325 79.6) (width 0.6) (layer "B.Cu") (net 16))
 (segment (start 118.37 79.6) (end 134.245 79.6) (width 0.6) (layer "B.Cu") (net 16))
 (segment (start 145.04 90.395) (end 145.675 89.76) (width 0.3) (layer "F.Cu") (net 17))
 (segment (start 145.04 93.57) (end 145.04 90.395) (width 0.3) (layer "F.Cu") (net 17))
 (segment (start 145.675 84.045) (end 139.325 77.695) (width 0.3) (layer "F.Cu") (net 17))
 (segment (start 145.675 89.76) (end 145.675 84.045) (width 0.3) (layer "F.Cu") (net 17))
 (segment (start 139.325 77.695) (end 139.325 71.98) (width 0.3) (layer "F.Cu") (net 17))
 (via (at 145.04 93.57) (size 0.6) (drill 0.3) (layers "F.Cu" "B.Cu") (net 17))
 (segment (start 139.325 75.155) (end 139.325 71.98) (width 0.2) (layer "B.Cu") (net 17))
 (segment (start 145.04 100) (end 145.04 93.57) (width 0.3) (layer "B.Cu") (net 17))
 (segment (start 124.72 91.665) (end 126.625 93.57) (width 0.3) (layer "F.Cu") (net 21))
 (segment (start 149.485 71.98) (end 149.485 70.075) (width 0.3) (layer "F.Cu") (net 21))
 (segment (start 126.625 93.57) (end 128.53 93.57) (width 0.3) (layer "F.Cu") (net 21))
 (segment (start 130.435 76.425) (end 124.72 82.14) (width 0.3) (layer "F.Cu") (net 21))
 (segment (start 149.485 77.695) (end 156.47 84.68) (width 0.4) (layer "F.Cu") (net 21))
 (segment (start 128.53 93.57) (end 129.8 94.84) (width 0.3) (layer "F.Cu") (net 21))
 (segment (start 129.8 94.84) (end 129.8 100) (width 0.3) (layer "F.Cu") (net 21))
 (segment (start 124.72 82.14) (end 124.72 91.665) (width 0.3) (layer "F.Cu") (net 21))
 (segment (start 156.47 84.68) (end 163.455 84.68) (width 0.4) (layer "F.Cu") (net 21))
 (segment (start 130.435 70.075) (end 130.435 76.425) (width 0.3) (layer "F.Cu") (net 21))
 (segment (start 163.455 84.68) (end 163.455 80.87) (width 0.4) (layer "F.Cu") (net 21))
 (segment (start 149.485 70.075) (end 148.215 68.805) (width 0.3) (layer "F.Cu") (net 21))
 (segment (start 131.705 68.805) (end 130.435 70.075) (width 0.3) (layer "F.Cu") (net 21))
 (segment (start 148.215 68.805) (end 131.705 68.805) (width 0.3) (layer "F.Cu") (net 21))
 (segment (start 149.485 71.98) (end 149.485 77.695) (width 0.4) (layer "F.Cu") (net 21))
 (segment (start 150.12 93.2525) (end 155.2 93.2525) (width 0.3) (layer "F.Cu") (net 8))
 (segment (start 150.755 85.315) (end 150.755 93.2525) (width 0.3) (layer "F.Cu") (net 8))
 (segment (start 140.595 85.315) (end 144.405 85.315) (width 0.3) (layer "F.Cu") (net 8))
 (via (at 150.12 93.2525) (size 0.6) (drill 0.3) (layers "F.Cu" "B.Cu") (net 8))
 (via (at 144.405 85.315) (size 0.6) (drill 0.3) (layers "F.Cu" "B.Cu") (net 8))
 (via (at 155.2 93.2525) (size 0.6) (drill 0.3) (layers "F.Cu" "B.Cu") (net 8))
 (via (at 140.595 85.315) (size 0.6) (drill 0.3) (layers "F.Cu" "B.Cu") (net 8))
 (via (at 150.755 85.315) (size 0.6) (drill 0.3) (layers "F.Cu" "B.Cu") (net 8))
 (segment (start 155.2 100) (end 155.2 93.2525) (width 0.3) (layer "B.Cu") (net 8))
 (segment (start 139.325 85.315) (end 139.325 87.22) (width 0.3) (layer "B.Cu") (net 8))
 (segment (start 139.325 85.315) (end 140.595 85.315) (width 0.3) (layer "B.Cu") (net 8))
 (segment (start 150.12 100) (end 150.12 93.2525) (width 0.3) (layer "B.Cu") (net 8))
 (segment (start 144.405 85.315) (end 150.755 85.315) (width 0.3) (layer "B.Cu") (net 8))
 (segment (start 139.325 84.045) (end 139.325 85.315) (width 0.3) (layer "B.Cu") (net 8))
 (segment (start 134.88 92.3) (end 134.88 100) (width 0.3) (layer "F.Cu") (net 25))
 (segment (start 118.37 87.855) (end 118.37 85.875002) (width 0.3) (layer "F.Cu") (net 25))
 (segment (start 134.245 91.665) (end 134.88 92.3) (width 0.3) (layer "F.Cu") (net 25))
 (segment (start 126.625 91.665) (end 134.245 91.665) (width 0.3) (layer "F.Cu") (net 25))
 (via (at 118.37 87.855) (size 0.6) (drill 0.3) (layers "F.Cu" "B.Cu") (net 25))
 (via (at 126.625 91.665) (size 0.6) (drill 0.3) (layers "F.Cu" "B.Cu") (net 25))
 (segment (start 118.37 87.855) (end 122.18 91.665) (width 0.3) (layer "B.Cu") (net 25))
 (segment (start 122.18 91.665) (end 126.625 91.665) (width 0.3) (layer "B.Cu") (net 25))
 (segment (start 128.53 90.395) (end 131.705 90.395) (width 0.3) (layer "F.Cu") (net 4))
 (via (at 128.53 90.395) (size 0.6) (drill 0.3) (layers "F.Cu" "B.Cu") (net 4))
 (via (at 131.705 90.395) (size 0.6) (drill 0.3) (layers "F.Cu" "B.Cu") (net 4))
 (segment (start 127.26 93.57) (end 127.26 100) (width 0.3) (layer "B.Cu") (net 4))
 (segment (start 128.53 90.395) (end 128.53 92.3) (width 0.3) (layer "B.Cu") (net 4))
 (segment (start 132.34 89.76) (end 147.58 89.76) (width 0.3) (layer "B.Cu") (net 4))
 (segment (start 128.53 92.3) (end 127.26 93.57) (width 0.3) (layer "B.Cu") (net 4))
 (segment (start 131.705 90.395) (end 132.34 89.76) (width 0.3) (layer "B.Cu") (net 4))
 (segment (start 147.58 89.76) (end 149.485 87.855) (width 0.3) (layer "B.Cu") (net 4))
 (segment (start 151.39 91.03) (end 136.15 91.03) (width 0.3) (layer "B.Cu") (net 2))
 (segment (start 154.565 87.855) (end 151.39 91.03) (width 0.3) (layer "B.Cu") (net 2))
 (segment (start 134.88 92.3) (end 134.88 100) (width 0.3) (layer "B.Cu") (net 2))
 (segment (start 136.15 91.03) (end 134.88 92.3) (width 0.3) (layer "B.Cu") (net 2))
 (segment (start 133.61 90.395) (end 149.485 90.395) (width 0.3) (layer "B.Cu") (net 3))
 (segment (start 132.34 91.665) (end 133.61 90.395) (width 0.3) (layer "B.Cu") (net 3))
 (segment (start 132.34 100) (end 132.34 91.665) (width 0.3) (layer "B.Cu") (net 3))
 (segment (start 152.025 87.855) (end 152.025 87.22) (width 0.3) (layer "B.Cu") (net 3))
 (segment (start 149.485 90.395) (end 152.025 87.855) (width 0.3) (layer "B.Cu") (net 3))
 (segment (start 134.245 84.105) (end 134.245 87.22) (width 0.3) (layer "B.Cu") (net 10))
 (segment (start 157.4225 82.4575) (end 160.28 85.315) (width 0.3) (layer "B.Cu") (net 10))
 (segment (start 160.28 85.315) (end 164.884999 85.315) (width 0.3) (layer "B.Cu") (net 10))
 (segment (start 134.245 84.105) (end 135.8925 82.4575) (width 0.3) (layer "B.Cu") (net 10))
 (segment (start 135.8925 82.4575) (end 157.4225 82.4575) (width 0.3) (layer "B.Cu") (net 10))
 (segment (start 164.884999 85.315) (end 165.995 84.204999) (width 0.3) (layer "B.Cu") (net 10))
 (segment (start 165.995 84.204999) (end 165.995 80.87) (width 0.3) (layer "B.Cu") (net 10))
 (segment (start 152.025 77.695) (end 157.74 83.41) (width 0.4) (layer "F.Cu") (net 22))
 (segment (start 160.915 83.41) (end 160.915 80.87) (width 0.4) (layer "F.Cu") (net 22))
 (segment (start 152.025 71.98) (end 152.025 77.695) (width 0.4) (layer "F.Cu") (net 22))
 (segment (start 157.74 83.41) (end 160.915 83.41) (width 0.4) (layer "F.Cu") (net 22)))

